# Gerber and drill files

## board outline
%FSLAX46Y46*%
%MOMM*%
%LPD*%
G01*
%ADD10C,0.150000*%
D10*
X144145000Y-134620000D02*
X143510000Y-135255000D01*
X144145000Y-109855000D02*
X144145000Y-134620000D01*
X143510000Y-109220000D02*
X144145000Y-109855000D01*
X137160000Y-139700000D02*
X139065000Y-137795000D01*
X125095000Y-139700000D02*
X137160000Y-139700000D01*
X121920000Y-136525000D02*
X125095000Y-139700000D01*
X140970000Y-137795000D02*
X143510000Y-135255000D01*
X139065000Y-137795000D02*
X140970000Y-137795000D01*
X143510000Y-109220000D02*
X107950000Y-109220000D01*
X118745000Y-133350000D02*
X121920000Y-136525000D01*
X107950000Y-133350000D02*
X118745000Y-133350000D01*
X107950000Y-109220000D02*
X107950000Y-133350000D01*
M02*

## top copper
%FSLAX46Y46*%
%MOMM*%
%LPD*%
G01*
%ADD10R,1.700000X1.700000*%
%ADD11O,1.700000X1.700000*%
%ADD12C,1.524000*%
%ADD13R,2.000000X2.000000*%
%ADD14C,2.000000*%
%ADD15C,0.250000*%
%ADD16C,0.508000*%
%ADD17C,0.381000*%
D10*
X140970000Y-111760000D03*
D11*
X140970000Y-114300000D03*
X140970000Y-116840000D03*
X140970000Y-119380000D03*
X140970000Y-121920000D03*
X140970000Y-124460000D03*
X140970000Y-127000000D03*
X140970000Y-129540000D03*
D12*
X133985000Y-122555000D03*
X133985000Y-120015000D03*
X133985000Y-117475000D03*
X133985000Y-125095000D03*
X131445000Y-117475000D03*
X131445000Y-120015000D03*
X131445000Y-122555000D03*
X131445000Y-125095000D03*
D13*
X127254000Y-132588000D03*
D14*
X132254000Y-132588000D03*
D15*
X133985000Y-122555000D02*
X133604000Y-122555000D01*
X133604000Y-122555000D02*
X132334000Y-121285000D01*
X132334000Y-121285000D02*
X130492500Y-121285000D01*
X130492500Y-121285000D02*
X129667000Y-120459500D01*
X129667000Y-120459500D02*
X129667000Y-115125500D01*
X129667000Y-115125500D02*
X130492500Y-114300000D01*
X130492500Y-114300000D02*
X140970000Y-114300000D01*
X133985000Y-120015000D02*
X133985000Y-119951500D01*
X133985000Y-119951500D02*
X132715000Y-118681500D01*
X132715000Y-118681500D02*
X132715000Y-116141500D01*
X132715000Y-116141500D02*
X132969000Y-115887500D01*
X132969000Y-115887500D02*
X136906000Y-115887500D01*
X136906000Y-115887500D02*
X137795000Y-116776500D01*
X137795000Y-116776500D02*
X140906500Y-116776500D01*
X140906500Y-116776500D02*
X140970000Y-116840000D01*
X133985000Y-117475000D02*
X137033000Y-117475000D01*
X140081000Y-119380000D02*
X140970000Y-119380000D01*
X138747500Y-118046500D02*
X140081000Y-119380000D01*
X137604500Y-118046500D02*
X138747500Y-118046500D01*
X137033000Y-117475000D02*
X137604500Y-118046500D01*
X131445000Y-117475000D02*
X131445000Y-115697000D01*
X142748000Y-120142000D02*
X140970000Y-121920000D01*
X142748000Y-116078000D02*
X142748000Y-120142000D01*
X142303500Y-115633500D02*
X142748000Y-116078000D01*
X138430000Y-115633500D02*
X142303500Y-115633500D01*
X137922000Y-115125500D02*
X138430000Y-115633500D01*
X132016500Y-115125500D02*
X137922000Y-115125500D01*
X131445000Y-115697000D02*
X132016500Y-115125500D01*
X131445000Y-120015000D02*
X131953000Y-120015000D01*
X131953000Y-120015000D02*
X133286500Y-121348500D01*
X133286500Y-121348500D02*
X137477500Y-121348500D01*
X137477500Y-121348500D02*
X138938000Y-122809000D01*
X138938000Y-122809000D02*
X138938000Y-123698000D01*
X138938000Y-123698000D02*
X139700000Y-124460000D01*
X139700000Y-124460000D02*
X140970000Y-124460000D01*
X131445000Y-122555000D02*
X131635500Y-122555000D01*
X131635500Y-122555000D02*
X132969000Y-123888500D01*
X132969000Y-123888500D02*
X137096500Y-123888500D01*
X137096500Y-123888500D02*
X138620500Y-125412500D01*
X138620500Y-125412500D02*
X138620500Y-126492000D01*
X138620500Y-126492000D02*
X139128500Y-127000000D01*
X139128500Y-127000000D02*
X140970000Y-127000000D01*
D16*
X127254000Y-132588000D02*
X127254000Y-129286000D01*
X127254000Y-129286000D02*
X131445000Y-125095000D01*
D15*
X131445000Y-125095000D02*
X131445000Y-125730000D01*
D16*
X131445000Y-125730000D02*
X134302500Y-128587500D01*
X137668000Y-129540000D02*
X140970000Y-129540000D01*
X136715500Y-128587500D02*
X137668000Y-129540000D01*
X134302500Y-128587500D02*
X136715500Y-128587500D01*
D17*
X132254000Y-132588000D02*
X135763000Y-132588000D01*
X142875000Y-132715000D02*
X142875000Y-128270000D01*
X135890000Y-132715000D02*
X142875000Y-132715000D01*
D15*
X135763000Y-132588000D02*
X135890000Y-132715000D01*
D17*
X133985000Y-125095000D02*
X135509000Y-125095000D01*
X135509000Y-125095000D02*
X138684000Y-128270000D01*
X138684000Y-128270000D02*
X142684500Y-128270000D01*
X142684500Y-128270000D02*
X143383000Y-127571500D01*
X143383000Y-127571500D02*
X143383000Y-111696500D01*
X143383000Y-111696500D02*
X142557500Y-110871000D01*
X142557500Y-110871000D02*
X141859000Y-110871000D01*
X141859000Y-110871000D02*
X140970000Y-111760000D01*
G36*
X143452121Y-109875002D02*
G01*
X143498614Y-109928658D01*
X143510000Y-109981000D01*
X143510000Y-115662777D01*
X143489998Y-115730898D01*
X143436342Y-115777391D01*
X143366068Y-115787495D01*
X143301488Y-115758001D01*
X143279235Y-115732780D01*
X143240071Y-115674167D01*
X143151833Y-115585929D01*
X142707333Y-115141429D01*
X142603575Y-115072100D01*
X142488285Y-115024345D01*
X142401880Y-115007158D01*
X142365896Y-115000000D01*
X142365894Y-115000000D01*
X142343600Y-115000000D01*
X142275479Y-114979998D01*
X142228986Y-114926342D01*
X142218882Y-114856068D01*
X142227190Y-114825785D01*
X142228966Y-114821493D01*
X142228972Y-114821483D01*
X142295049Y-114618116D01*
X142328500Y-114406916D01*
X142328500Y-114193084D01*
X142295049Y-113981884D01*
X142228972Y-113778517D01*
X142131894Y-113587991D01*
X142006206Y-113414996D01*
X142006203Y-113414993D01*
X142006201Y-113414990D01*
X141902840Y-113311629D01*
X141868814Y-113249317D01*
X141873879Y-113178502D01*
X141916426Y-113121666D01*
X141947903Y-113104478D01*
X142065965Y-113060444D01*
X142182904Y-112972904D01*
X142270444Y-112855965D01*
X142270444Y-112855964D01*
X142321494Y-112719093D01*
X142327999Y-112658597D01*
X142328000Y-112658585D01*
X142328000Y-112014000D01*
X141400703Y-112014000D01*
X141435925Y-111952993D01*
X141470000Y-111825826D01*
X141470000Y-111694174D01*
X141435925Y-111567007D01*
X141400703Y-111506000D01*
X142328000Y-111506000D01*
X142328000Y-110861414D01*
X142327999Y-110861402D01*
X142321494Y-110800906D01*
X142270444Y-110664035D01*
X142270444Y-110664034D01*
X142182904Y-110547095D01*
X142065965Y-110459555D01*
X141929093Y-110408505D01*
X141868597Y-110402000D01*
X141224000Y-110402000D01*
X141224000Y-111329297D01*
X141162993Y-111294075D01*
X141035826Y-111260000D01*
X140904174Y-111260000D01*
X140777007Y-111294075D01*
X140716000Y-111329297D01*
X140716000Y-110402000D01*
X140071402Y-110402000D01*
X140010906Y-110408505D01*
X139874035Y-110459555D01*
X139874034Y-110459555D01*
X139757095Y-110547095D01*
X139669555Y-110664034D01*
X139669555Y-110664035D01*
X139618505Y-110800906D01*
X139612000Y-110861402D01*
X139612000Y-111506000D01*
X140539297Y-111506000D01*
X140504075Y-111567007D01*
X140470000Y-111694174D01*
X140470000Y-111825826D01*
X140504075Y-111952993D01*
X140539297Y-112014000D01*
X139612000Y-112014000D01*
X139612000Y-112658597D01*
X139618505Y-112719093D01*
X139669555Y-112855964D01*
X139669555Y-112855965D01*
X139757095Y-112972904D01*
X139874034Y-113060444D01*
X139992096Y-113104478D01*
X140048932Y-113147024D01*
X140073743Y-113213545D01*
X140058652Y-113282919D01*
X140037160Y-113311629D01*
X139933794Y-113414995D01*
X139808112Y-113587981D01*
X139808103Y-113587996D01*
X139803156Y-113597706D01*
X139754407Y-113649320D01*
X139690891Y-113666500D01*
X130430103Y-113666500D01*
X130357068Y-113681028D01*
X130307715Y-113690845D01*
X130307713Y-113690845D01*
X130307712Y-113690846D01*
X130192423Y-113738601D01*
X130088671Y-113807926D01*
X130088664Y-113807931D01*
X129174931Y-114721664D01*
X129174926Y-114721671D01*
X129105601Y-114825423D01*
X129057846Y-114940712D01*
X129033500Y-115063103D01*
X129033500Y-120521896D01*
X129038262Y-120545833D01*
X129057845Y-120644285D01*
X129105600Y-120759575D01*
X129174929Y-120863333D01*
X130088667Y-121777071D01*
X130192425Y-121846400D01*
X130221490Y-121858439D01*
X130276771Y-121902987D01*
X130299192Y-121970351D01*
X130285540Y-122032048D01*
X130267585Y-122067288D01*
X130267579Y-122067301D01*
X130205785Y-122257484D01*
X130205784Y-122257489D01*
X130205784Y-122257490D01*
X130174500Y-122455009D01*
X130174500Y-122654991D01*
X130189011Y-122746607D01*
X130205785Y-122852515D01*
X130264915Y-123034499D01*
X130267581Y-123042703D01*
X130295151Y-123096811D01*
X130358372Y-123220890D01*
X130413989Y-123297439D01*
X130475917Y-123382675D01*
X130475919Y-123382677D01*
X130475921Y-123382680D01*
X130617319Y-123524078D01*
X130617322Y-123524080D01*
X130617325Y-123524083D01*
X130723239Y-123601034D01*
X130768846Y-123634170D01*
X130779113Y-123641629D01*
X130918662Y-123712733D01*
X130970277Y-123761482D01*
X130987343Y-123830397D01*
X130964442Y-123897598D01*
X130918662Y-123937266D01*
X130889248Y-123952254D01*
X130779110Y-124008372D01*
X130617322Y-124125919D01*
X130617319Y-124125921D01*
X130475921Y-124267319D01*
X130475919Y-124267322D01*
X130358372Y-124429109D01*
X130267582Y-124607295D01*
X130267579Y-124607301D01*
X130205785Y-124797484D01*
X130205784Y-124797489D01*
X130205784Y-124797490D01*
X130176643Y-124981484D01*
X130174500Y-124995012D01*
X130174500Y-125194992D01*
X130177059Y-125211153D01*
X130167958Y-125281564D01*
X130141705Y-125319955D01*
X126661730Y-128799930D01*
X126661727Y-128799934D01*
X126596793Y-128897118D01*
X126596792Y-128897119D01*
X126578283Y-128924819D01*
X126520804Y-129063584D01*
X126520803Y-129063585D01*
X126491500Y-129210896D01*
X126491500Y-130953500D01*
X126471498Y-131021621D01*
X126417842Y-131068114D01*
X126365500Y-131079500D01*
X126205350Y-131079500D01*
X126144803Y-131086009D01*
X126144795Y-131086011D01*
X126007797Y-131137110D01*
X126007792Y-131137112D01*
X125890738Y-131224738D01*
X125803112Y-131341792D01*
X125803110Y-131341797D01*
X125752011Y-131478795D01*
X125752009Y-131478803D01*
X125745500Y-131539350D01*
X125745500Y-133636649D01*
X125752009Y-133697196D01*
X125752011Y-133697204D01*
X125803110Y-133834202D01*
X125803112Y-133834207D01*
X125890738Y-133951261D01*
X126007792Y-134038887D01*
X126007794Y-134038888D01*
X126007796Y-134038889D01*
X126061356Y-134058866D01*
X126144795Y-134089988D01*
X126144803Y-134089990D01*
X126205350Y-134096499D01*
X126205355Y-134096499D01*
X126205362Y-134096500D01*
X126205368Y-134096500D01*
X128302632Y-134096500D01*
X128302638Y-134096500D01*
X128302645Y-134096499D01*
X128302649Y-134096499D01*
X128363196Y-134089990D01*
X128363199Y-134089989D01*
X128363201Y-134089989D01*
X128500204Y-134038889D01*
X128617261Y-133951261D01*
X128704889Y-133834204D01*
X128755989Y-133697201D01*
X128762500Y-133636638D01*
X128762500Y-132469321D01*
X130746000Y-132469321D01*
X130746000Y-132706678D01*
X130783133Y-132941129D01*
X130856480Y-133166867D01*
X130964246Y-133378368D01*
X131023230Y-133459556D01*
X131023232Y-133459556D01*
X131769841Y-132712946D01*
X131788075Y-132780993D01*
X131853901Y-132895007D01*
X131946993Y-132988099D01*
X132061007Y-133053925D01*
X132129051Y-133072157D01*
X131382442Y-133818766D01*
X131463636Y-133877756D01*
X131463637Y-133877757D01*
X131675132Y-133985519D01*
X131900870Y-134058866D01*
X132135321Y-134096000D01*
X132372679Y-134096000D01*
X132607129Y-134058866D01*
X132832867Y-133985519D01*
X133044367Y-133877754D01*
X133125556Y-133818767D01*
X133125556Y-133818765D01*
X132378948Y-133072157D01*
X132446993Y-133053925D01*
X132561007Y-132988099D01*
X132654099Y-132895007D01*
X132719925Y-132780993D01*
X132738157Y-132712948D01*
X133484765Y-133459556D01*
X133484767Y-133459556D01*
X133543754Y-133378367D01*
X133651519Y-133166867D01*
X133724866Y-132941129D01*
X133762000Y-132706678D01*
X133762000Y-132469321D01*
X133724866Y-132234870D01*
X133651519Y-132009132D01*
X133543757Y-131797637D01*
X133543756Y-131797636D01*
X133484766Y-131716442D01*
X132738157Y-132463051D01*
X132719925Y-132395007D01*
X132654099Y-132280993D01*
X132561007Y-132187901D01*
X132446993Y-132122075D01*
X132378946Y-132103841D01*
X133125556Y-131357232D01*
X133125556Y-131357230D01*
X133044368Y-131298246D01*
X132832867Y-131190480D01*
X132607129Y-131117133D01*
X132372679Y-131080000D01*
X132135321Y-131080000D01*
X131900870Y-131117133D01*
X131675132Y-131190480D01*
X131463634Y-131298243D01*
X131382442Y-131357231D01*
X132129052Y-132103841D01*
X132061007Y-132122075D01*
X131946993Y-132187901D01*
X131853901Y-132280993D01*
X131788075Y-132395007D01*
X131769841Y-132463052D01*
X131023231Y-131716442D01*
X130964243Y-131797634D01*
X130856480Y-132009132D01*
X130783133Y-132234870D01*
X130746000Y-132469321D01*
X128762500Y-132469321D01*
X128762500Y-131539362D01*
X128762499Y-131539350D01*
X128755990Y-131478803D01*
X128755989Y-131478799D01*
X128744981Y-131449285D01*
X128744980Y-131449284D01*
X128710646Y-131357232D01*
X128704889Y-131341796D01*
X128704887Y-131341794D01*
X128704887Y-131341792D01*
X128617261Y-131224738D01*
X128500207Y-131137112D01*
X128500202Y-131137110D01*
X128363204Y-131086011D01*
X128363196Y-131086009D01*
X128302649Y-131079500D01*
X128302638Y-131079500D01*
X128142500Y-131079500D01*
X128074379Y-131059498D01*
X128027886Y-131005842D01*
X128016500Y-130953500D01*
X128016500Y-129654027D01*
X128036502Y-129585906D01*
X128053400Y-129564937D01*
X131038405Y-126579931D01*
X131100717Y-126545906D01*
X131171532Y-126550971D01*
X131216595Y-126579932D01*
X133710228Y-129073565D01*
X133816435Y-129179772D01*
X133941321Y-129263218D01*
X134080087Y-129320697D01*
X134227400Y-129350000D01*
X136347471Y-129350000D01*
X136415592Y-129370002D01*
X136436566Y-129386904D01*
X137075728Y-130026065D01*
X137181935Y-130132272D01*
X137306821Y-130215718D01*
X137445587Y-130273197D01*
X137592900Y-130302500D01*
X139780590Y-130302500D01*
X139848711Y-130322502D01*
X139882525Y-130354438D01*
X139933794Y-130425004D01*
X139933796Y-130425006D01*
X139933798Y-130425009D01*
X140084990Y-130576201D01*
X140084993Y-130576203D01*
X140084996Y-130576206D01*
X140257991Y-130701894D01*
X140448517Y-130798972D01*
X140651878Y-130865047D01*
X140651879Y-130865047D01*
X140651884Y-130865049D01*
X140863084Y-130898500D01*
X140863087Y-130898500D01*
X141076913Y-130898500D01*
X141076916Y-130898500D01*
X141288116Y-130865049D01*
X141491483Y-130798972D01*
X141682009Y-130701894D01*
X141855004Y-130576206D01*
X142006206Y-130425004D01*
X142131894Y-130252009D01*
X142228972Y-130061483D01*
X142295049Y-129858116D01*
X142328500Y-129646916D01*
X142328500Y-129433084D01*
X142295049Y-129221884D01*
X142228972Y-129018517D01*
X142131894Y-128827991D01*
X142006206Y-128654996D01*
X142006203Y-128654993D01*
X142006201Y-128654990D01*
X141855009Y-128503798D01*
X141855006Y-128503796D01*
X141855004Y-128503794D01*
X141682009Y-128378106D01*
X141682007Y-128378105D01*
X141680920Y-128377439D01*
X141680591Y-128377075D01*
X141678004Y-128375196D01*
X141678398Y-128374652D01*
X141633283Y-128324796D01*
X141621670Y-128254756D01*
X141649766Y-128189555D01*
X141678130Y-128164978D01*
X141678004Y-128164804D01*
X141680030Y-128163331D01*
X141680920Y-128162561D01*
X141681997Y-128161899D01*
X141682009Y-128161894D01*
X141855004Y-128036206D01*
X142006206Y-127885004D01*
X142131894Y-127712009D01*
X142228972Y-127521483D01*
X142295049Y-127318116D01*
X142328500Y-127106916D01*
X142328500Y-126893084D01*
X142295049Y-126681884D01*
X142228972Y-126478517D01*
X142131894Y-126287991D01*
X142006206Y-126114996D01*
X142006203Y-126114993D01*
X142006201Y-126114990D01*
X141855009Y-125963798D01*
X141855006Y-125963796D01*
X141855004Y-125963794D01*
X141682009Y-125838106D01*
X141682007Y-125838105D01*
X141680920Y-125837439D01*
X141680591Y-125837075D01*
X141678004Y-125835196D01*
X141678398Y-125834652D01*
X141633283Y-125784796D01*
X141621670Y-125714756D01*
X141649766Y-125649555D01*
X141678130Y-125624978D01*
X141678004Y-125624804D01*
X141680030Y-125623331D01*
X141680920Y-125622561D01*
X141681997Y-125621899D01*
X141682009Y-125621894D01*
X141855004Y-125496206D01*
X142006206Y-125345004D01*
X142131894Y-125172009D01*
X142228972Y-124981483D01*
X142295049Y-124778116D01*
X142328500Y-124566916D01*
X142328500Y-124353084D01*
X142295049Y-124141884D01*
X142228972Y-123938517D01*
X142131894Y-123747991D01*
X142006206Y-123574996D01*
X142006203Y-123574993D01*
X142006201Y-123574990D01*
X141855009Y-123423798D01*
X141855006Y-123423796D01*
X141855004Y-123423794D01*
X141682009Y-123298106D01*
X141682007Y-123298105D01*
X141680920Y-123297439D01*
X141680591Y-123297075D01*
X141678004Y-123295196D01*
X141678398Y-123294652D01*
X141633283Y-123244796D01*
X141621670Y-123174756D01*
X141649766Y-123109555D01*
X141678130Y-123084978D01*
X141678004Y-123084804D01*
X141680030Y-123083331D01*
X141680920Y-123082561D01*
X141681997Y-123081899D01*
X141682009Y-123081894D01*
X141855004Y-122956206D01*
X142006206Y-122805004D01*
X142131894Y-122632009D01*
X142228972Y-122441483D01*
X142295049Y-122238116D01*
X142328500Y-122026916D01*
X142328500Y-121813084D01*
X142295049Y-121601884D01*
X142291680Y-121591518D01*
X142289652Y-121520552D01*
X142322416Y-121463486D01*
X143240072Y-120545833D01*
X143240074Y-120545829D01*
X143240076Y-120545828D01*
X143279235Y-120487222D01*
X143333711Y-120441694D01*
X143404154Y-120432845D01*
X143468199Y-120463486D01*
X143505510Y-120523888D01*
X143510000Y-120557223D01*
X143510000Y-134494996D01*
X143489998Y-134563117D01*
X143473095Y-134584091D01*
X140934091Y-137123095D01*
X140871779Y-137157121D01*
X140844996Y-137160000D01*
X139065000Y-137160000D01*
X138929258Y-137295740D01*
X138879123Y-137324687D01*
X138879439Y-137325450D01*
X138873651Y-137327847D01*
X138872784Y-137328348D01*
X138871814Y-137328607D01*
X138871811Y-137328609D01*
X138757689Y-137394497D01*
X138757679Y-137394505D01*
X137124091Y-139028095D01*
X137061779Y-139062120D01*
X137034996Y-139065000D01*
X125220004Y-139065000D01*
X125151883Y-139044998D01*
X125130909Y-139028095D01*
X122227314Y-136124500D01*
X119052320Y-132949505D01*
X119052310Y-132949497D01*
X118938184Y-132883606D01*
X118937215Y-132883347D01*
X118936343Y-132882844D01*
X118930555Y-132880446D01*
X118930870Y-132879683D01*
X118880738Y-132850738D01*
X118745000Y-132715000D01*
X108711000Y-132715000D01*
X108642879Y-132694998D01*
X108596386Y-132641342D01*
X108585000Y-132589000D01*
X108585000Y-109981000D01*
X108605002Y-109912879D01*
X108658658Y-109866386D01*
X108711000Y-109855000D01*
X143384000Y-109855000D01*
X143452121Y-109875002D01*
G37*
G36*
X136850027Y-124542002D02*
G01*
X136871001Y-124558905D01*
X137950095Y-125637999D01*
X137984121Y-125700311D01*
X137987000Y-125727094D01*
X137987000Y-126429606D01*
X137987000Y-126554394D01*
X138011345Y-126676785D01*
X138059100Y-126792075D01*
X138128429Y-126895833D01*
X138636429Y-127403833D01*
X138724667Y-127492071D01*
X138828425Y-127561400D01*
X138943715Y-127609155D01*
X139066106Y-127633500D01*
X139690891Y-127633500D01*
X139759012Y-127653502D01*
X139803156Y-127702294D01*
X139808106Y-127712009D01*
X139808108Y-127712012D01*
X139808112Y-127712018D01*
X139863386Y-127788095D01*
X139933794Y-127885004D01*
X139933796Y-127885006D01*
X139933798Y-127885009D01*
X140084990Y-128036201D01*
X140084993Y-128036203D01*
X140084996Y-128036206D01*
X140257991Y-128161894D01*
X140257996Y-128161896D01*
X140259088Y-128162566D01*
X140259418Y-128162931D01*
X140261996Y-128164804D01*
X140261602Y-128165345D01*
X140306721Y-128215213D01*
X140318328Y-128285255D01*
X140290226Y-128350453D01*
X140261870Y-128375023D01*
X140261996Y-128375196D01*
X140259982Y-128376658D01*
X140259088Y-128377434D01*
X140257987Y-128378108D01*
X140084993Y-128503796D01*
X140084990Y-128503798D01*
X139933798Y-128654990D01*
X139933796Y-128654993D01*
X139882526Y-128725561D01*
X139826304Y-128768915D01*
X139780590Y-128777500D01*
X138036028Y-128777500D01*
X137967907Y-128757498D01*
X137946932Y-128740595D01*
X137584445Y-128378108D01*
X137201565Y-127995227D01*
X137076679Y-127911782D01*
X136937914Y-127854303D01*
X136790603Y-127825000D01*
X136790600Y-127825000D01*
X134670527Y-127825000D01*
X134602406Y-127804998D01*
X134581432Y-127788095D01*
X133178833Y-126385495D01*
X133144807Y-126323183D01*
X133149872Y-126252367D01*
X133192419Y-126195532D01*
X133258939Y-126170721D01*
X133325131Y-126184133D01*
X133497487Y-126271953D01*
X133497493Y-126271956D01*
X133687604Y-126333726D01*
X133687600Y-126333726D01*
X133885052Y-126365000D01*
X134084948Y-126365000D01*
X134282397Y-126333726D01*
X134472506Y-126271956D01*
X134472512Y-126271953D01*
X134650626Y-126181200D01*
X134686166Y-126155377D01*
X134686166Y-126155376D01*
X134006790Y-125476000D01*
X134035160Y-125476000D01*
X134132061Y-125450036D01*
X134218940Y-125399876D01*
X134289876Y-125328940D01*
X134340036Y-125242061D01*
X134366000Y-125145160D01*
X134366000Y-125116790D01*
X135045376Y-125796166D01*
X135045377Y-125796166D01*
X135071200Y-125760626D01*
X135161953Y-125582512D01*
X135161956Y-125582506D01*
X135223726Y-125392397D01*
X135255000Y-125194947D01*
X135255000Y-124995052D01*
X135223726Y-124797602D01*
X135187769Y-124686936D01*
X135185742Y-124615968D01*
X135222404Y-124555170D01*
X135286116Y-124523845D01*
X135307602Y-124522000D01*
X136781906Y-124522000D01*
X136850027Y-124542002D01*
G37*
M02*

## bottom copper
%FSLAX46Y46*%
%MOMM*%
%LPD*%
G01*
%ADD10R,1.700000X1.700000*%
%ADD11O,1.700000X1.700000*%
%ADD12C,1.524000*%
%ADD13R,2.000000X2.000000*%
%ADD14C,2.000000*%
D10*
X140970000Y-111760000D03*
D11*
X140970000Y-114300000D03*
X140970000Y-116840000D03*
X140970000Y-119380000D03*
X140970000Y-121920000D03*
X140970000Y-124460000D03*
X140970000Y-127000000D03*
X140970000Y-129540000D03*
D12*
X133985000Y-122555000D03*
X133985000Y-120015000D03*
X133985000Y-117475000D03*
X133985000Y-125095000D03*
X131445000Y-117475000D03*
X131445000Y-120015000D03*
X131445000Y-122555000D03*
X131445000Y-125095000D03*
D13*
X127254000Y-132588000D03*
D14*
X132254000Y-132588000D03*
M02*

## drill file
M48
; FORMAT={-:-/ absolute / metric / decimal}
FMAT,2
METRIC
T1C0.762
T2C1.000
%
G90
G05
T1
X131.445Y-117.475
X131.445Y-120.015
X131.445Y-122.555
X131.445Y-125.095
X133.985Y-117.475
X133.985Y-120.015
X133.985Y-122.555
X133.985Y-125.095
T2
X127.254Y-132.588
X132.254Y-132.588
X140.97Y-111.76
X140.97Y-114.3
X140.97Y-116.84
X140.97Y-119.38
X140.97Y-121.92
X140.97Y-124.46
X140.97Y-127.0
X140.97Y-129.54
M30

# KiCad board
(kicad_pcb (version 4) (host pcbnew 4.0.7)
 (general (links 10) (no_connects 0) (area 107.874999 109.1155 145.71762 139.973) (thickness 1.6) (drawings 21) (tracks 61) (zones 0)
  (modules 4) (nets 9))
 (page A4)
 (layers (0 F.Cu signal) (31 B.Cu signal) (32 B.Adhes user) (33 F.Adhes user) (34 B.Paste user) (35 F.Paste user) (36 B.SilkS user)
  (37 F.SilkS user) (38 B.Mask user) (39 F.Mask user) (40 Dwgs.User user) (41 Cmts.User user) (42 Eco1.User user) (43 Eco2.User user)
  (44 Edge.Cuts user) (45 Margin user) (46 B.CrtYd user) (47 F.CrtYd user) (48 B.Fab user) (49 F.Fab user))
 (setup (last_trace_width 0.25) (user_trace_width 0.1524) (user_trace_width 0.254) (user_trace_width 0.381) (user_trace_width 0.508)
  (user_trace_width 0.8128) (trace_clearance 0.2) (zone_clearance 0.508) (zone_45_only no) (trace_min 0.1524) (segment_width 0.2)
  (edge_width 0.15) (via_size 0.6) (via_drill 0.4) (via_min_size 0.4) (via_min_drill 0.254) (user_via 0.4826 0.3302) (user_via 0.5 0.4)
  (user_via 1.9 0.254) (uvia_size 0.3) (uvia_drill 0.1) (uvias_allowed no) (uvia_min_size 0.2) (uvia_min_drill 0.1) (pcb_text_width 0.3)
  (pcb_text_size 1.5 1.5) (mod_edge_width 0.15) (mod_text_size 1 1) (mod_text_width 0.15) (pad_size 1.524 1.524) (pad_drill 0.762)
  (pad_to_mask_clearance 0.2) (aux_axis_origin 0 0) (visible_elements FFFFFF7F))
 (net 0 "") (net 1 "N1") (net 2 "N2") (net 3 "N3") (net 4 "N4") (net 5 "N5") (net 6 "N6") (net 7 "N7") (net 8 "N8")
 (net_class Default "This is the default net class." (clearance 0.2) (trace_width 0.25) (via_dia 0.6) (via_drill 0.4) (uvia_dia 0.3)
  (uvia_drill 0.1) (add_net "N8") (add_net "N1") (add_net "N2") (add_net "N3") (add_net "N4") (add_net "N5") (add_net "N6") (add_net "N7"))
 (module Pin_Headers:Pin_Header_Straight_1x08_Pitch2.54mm (layer F.Cu) (at 140.97 111.76)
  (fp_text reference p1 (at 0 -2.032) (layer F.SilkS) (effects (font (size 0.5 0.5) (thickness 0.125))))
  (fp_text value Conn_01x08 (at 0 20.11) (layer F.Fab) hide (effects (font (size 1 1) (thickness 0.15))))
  (pad 1 thru_hole rect (at 0 0) (size 1.7 1.7) (drill 1) (layers *.Cu *.Mask) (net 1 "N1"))
  (pad 2 thru_hole oval (at 0 2.54) (size 1.7 1.7) (drill 1) (layers *.Cu *.Mask) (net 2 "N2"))
  (pad 3 thru_hole oval (at 0 5.08) (size 1.7 1.7) (drill 1) (layers *.Cu *.Mask) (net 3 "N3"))
  (pad 4 thru_hole oval (at 0 7.62) (size 1.7 1.7) (drill 1) (layers *.Cu *.Mask) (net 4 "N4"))
  (pad 5 thru_hole oval (at 0 10.16) (size 1.7 1.7) (drill 1) (layers *.Cu *.Mask) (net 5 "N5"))
  (pad 6 thru_hole oval (at 0 12.7) (size 1.7 1.7) (drill 1) (layers *.Cu *.Mask) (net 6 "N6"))
  (pad 7 thru_hole oval (at 0 15.24) (size 1.7 1.7) (drill 1) (layers *.Cu *.Mask) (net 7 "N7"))
  (pad 8 thru_hole oval (at 0 17.78) (size 1.7 1.7) (drill 1) (layers *.Cu *.Mask) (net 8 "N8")))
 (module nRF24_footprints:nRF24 (layer F.Cu) (at 123.825 123.825)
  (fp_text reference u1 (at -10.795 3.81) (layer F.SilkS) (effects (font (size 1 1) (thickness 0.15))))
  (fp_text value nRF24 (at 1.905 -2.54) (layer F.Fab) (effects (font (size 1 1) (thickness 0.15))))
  (pad 1 thru_hole circle (at 10.16 -1.27) (size 1.524 1.524) (drill 0.762) (layers *.Cu *.Mask) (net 2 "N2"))
  (pad 2 thru_hole circle (at 10.16 -3.81) (size 1.524 1.524) (drill 0.762) (layers *.Cu *.Mask) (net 3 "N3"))
  (pad 3 thru_hole circle (at 10.16 -6.35) (size 1.524 1.524) (drill 0.762) (layers *.Cu *.Mask) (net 4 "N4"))
  (pad 0 thru_hole circle (at 10.16 1.27) (size 1.524 1.524) (drill 0.762) (layers *.Cu *.Mask) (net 1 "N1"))
  (pad 4 thru_hole circle (at 7.62 -6.35) (size 1.524 1.524) (drill 0.762) (layers *.Cu *.Mask) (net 5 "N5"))
  (pad 5 thru_hole circle (at 7.62 -3.81) (size 1.524 1.524) (drill 0.762) (layers *.Cu *.Mask) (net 6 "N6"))
  (pad 6 thru_hole circle (at 7.62 -1.27) (size 1.524 1.524) (drill 0.762) (layers *.Cu *.Mask) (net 7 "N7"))
  (pad 7 thru_hole circle (at 7.62 1.27) (size 1.524 1.524) (drill 0.762) (layers *.Cu *.Mask) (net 8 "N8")))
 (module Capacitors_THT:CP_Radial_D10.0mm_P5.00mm (layer F.Cu) (at 127.254 132.588)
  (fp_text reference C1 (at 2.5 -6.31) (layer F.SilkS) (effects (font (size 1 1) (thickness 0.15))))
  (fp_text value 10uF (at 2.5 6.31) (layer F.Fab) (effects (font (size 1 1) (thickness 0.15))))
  (pad 1 thru_hole rect (at 0 0) (size 2 2) (drill 1) (layers *.Cu *.Mask) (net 8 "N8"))
  (pad 2 thru_hole circle (at 5 0) (size 2 2) (drill 1) (layers *.Cu *.Mask) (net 1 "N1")))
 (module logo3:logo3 (layer F.Cu) (at 120.142 113.284)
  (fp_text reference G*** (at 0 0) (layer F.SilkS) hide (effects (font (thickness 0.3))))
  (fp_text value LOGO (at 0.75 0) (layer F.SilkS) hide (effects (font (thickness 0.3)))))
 (gr_line (start 144.145 134.62) (end 143.51 135.255) (angle 90) (layer Edge.Cuts) (width 0.15))
 (gr_line (start 144.145 109.855) (end 144.145 134.62) (angle 90) (layer Edge.Cuts) (width 0.15))
 (gr_line (start 143.51 109.22) (end 144.145 109.855) (angle 90) (layer Edge.Cuts) (width 0.15))
 (gr_line (start 137.16 139.7) (end 139.065 137.795) (angle 90) (layer Edge.Cuts) (width 0.15))
 (gr_line (start 125.095 139.7) (end 137.16 139.7) (angle 90) (layer Edge.Cuts) (width 0.15))
 (gr_line (start 121.92 136.525) (end 125.095 139.7) (angle 90) (layer Edge.Cuts) (width 0.15))
 (gr_line (start 140.97 137.795) (end 143.51 135.255) (angle 90) (layer Edge.Cuts) (width 0.15))
 (gr_line (start 139.065 137.795) (end 140.97 137.795) (angle 90) (layer Edge.Cuts) (width 0.15))
 (gr_line (start 143.51 109.22) (end 107.95 109.22) (angle 90) (layer Edge.Cuts) (width 0.15))
 (gr_line (start 118.745 133.35) (end 121.92 136.525) (angle 90) (layer Edge.Cuts) (width 0.15))
 (gr_line (start 107.95 133.35) (end 118.745 133.35) (angle 90) (layer Edge.Cuts) (width 0.15))
 (gr_line (start 107.95 109.22) (end 107.95 133.35) (angle 90) (layer Edge.Cuts) (width 0.15))
 (segment (start 133.985 122.555) (end 133.604 122.555) (width 0.25) (layer F.Cu) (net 2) (status 30))
 (segment (start 133.604 122.555) (end 132.334 121.285) (width 0.25) (layer F.Cu) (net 2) (status 10))
 (segment (start 132.334 121.285) (end 130.4925 121.285) (width 0.25) (layer F.Cu) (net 2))
 (segment (start 130.4925 121.285) (end 129.667 120.4595) (width 0.25) (layer F.Cu) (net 2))
 (segment (start 129.667 120.4595) (end 129.667 115.1255) (width 0.25) (layer F.Cu) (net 2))
 (segment (start 129.667 115.1255) (end 130.4925 114.3) (width 0.25) (layer F.Cu) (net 2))
 (segment (start 130.4925 114.3) (end 140.97 114.3) (width 0.25) (layer F.Cu) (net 2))
 (segment (start 133.985 120.015) (end 133.985 119.9515) (width 0.25) (layer F.Cu) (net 3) (status 30))
 (segment (start 133.985 119.9515) (end 132.715 118.6815) (width 0.25) (layer F.Cu) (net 3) (status 10))
 (segment (start 132.715 118.6815) (end 132.715 116.1415) (width 0.25) (layer F.Cu) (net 3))
 (segment (start 132.715 116.1415) (end 132.969 115.8875) (width 0.25) (layer F.Cu) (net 3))
 (segment (start 132.969 115.8875) (end 136.906 115.8875) (width 0.25) (layer F.Cu) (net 3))
 (segment (start 136.906 115.8875) (end 137.795 116.7765) (width 0.25) (layer F.Cu) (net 3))
 (segment (start 137.795 116.7765) (end 140.9065 116.7765) (width 0.25) (layer F.Cu) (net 3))
 (segment (start 140.9065 116.7765) (end 140.97 116.84) (width 0.25) (layer F.Cu) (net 3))
 (segment (start 133.985 117.475) (end 137.033 117.475) (width 0.25) (layer F.Cu) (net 4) (status 10))
 (segment (start 140.081 119.38) (end 140.97 119.38) (width 0.25) (layer F.Cu) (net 4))
 (segment (start 138.7475 118.0465) (end 140.081 119.38) (width 0.25) (layer F.Cu) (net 4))
 (segment (start 137.6045 118.0465) (end 138.7475 118.0465) (width 0.25) (layer F.Cu) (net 4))
 (segment (start 137.033 117.475) (end 137.6045 118.0465) (width 0.25) (layer F.Cu) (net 4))
 (segment (start 131.445 117.475) (end 131.445 115.697) (width 0.25) (layer F.Cu) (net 5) (status 10))
 (segment (start 142.748 120.142) (end 140.97 121.92) (width 0.25) (layer F.Cu) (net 5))
 (segment (start 142.748 116.078) (end 142.748 120.142) (width 0.25) (layer F.Cu) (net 5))
 (segment (start 142.3035 115.6335) (end 142.748 116.078) (width 0.25) (layer F.Cu) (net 5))
 (segment (start 138.43 115.6335) (end 142.3035 115.6335) (width 0.25) (layer F.Cu) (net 5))
 (segment (start 137.922 115.1255) (end 138.43 115.6335) (width 0.25) (layer F.Cu) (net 5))
 (segment (start 132.0165 115.1255) (end 137.922 115.1255) (width 0.25) (layer F.Cu) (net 5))
 (segment (start 131.445 115.697) (end 132.0165 115.1255) (width 0.25) (layer F.Cu) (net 5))
 (segment (start 131.445 120.015) (end 131.953 120.015) (width 0.25) (layer F.Cu) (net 6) (status 30))
 (segment (start 131.953 120.015) (end 133.2865 121.3485) (width 0.25) (layer F.Cu) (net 6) (status 10))
 (segment (start 133.2865 121.3485) (end 137.4775 121.3485) (width 0.25) (layer F.Cu) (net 6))
 (segment (start 137.4775 121.3485) (end 138.938 122.809) (width 0.25) (layer F.Cu) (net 6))
 (segment (start 138.938 122.809) (end 138.938 123.698) (width 0.25) (layer F.Cu) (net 6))
 (segment (start 138.938 123.698) (end 139.7 124.46) (width 0.25) (layer F.Cu) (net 6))
 (segment (start 139.7 124.46) (end 140.97 124.46) (width 0.25) (layer F.Cu) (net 6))
 (segment (start 131.445 122.555) (end 131.6355 122.555) (width 0.25) (layer F.Cu) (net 7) (status 30))
 (segment (start 131.6355 122.555) (end 132.969 123.8885) (width 0.25) (layer F.Cu) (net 7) (status 10))
 (segment (start 132.969 123.8885) (end 137.0965 123.8885) (width 0.25) (layer F.Cu) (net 7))
 (segment (start 137.0965 123.8885) (end 138.6205 125.4125) (width 0.25) (layer F.Cu) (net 7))
 (segment (start 138.6205 125.4125) (end 138.6205 126.492) (width 0.25) (layer F.Cu) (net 7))
 (segment (start 138.6205 126.492) (end 139.1285 127) (width 0.25) (layer F.Cu) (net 7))
 (segment (start 139.1285 127) (end 140.97 127) (width 0.25) (layer F.Cu) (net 7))
 (segment (start 127.254 132.588) (end 127.254 129.286) (width 0.508) (layer F.Cu) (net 8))
 (segment (start 127.254 129.286) (end 131.445 125.095) (width 0.508) (layer F.Cu) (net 8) (status 20))
 (segment (start 131.445 125.095) (end 131.445 125.73) (width 0.25) (layer F.Cu) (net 8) (status 30))
 (segment (start 131.445 125.73) (end 134.3025 128.5875) (width 0.508) (layer F.Cu) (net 8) (status 10))
 (segment (start 137.668 129.54) (end 140.97 129.54) (width 0.508) (layer F.Cu) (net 8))
 (segment (start 136.7155 128.5875) (end 137.668 129.54) (width 0.508) (layer F.Cu) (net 8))
 (segment (start 134.3025 128.5875) (end 136.7155 128.5875) (width 0.508) (layer F.Cu) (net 8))
 (segment (start 132.254 132.588) (end 135.763 132.588) (width 0.381) (layer F.Cu) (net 1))
 (segment (start 142.875 132.715) (end 142.875 128.27) (width 0.381) (layer F.Cu) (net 1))
 (segment (start 135.89 132.715) (end 142.875 132.715) (width 0.381) (layer F.Cu) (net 1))
 (segment (start 135.763 132.588) (end 135.89 132.715) (width 0.25) (layer F.Cu) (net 1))
 (segment (start 133.985 125.095) (end 135.509 125.095) (width 0.381) (layer F.Cu) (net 1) (status 10))
 (segment (start 135.509 125.095) (end 138.684 128.27) (width 0.381) (layer F.Cu) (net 1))
 (segment (start 138.684 128.27) (end 142.6845 128.27) (width 0.381) (layer F.Cu) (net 1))
 (segment (start 142.6845 128.27) (end 143.383 127.5715) (width 0.381) (layer F.Cu) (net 1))
 (segment (start 143.383 127.5715) (end 143.383 111.6965) (width 0.381) (layer F.Cu) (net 1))
 (segment (start 143.383 111.6965) (end 142.5575 110.871) (width 0.381) (layer F.Cu) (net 1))
 (segment (start 142.5575 110.871) (end 141.859 110.871) (width 0.381) (layer F.Cu) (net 1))
 (segment (start 141.859 110.871) (end 140.97 111.76) (width 0.381) (layer F.Cu) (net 1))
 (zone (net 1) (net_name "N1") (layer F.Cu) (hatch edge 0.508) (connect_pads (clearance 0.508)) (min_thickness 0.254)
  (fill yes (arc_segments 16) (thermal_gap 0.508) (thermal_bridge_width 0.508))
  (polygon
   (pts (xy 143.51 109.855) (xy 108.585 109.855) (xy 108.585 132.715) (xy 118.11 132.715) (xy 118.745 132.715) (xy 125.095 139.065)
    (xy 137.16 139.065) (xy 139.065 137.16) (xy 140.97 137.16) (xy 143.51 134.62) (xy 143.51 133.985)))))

